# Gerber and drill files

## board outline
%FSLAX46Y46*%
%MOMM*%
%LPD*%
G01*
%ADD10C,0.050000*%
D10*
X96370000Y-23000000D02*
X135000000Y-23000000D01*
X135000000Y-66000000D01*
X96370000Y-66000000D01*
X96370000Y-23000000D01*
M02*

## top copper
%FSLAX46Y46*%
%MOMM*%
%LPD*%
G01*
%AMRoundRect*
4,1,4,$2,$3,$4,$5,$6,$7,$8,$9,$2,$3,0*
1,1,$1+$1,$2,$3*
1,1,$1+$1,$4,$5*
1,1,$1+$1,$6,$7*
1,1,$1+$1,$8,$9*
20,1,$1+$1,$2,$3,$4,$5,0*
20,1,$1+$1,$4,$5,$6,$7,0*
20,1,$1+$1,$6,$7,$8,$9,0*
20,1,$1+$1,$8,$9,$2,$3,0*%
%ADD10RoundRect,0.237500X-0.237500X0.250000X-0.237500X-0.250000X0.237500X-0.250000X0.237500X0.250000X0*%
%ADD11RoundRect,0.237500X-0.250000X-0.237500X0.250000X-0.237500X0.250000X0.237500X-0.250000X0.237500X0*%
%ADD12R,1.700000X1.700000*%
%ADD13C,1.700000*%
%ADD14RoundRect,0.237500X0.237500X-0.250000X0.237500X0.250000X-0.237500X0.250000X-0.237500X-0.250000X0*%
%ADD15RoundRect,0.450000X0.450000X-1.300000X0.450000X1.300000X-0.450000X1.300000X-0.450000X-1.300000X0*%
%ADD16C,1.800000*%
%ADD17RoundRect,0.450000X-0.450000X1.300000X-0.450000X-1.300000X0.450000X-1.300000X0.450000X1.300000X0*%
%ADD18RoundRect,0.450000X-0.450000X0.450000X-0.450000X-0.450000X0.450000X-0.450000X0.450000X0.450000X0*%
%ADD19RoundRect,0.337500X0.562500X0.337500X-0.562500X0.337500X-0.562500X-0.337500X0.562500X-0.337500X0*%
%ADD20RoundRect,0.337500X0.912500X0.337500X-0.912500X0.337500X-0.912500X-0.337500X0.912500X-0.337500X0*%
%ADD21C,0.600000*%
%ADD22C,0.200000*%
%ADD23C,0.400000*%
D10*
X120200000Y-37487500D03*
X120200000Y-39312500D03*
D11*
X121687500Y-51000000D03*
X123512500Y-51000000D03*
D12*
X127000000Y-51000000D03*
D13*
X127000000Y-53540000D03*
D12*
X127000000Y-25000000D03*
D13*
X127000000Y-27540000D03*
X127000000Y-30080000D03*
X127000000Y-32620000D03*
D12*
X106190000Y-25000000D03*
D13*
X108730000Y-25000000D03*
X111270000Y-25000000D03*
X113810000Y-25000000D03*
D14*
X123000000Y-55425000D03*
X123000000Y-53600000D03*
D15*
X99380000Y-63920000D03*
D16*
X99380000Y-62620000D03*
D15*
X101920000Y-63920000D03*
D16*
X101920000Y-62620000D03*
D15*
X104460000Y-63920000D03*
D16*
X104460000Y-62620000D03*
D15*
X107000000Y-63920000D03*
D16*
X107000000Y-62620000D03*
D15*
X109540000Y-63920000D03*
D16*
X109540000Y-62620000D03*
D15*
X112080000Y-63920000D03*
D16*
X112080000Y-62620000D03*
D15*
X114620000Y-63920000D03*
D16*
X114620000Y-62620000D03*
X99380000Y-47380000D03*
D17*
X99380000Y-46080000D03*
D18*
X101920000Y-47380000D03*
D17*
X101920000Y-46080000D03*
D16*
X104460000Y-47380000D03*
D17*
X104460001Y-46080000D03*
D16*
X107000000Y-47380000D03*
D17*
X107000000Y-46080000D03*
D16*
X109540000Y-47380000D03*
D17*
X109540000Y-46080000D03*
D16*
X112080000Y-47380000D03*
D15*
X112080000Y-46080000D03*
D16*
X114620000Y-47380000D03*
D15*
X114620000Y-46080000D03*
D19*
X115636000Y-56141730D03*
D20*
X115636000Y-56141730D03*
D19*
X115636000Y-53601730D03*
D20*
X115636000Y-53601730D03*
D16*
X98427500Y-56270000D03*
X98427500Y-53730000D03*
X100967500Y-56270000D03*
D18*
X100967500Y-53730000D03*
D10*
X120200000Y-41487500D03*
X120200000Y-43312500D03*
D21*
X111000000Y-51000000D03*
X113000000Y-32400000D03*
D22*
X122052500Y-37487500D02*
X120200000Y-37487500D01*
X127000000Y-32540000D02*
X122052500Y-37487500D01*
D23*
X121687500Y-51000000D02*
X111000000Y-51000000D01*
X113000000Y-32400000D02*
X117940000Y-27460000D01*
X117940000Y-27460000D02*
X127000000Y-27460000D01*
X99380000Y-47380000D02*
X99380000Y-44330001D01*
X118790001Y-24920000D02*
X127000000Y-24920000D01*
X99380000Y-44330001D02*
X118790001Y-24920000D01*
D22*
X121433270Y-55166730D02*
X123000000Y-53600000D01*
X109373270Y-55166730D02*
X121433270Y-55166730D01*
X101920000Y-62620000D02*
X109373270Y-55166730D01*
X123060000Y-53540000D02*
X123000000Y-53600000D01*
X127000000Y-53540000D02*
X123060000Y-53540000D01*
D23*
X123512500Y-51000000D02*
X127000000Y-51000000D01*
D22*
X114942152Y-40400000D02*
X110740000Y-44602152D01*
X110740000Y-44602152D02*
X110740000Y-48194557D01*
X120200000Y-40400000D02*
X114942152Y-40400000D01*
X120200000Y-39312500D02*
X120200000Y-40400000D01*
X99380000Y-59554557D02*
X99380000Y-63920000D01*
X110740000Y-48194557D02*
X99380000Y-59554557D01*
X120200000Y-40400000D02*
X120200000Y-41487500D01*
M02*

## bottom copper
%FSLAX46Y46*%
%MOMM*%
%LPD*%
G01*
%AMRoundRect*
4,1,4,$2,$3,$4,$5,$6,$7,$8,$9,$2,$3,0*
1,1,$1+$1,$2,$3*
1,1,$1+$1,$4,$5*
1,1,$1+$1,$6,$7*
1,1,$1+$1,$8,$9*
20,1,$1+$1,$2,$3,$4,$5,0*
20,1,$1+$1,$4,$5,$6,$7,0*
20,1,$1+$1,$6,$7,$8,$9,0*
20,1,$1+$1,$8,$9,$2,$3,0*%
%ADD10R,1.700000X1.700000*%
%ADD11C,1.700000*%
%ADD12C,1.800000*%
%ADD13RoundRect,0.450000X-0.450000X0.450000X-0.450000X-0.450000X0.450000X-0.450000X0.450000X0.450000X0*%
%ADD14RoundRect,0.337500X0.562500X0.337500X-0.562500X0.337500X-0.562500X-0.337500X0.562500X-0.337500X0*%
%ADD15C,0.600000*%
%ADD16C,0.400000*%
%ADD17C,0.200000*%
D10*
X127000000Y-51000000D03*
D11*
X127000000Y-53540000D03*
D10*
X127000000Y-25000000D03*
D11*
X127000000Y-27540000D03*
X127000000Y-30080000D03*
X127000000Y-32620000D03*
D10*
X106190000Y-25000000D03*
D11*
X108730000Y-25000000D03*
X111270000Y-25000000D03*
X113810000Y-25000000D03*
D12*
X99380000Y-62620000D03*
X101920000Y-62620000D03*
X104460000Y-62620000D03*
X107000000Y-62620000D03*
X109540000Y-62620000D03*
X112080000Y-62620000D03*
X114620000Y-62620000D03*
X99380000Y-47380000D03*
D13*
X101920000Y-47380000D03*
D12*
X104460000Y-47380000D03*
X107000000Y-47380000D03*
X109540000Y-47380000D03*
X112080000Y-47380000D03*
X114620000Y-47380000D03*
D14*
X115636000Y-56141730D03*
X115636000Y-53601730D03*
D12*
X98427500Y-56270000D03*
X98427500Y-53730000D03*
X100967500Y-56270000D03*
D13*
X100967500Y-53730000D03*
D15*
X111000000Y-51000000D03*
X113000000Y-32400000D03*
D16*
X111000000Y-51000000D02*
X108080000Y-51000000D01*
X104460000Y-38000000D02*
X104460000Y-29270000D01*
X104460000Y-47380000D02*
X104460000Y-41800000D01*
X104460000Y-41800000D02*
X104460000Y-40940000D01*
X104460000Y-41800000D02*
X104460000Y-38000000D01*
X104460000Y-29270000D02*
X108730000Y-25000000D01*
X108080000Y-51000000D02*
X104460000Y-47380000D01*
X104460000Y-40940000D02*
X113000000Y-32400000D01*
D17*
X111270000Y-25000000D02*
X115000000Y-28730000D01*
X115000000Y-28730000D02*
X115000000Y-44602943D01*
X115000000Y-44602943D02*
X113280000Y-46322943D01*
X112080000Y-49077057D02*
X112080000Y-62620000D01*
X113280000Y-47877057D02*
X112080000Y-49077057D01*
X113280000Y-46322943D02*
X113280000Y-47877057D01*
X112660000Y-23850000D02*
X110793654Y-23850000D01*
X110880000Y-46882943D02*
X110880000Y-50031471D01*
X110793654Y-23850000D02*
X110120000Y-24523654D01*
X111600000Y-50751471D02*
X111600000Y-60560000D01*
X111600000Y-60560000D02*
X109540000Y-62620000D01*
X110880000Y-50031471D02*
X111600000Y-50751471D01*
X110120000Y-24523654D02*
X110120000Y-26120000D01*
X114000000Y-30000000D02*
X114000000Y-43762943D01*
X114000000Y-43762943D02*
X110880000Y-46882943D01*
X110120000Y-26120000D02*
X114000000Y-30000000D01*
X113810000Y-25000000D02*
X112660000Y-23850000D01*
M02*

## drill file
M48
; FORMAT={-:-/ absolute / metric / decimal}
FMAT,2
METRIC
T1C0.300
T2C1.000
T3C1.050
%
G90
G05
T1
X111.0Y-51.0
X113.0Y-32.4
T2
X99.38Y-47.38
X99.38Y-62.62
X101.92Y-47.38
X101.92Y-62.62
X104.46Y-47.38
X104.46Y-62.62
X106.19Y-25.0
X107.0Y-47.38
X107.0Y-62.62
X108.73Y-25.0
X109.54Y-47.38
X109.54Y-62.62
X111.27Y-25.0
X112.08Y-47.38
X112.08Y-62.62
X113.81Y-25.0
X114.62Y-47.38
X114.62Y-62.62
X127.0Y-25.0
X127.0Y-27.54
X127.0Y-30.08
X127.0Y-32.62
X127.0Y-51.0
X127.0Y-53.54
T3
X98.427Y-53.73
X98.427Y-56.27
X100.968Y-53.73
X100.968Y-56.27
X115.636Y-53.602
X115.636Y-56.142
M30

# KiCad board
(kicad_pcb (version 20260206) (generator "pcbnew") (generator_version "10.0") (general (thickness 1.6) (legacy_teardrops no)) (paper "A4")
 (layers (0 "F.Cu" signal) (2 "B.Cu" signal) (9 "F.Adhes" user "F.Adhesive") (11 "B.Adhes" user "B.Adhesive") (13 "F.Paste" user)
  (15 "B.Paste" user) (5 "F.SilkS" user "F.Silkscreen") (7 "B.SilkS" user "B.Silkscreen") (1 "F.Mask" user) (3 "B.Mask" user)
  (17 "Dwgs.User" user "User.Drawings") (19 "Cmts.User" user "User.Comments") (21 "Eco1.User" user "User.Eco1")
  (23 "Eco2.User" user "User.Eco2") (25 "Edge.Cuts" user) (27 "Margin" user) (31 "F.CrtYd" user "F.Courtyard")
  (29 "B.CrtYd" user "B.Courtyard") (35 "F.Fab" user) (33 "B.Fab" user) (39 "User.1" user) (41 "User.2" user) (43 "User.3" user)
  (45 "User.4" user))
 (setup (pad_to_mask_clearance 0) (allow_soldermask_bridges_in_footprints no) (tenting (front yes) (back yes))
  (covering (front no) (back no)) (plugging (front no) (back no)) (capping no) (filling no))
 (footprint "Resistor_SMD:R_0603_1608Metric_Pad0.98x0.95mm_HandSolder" (layer "F.Cu") (at 120.2 38.4 -90)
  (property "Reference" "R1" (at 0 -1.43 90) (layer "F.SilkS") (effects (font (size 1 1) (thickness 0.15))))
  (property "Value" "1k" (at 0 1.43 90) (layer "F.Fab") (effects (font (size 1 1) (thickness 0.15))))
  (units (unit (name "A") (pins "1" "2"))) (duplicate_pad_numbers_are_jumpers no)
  (pad "1" smd roundrect (at -0.9125 0 270) (size 0.975 0.95) (layers "F.Cu" "F.Mask" "F.Paste") (roundrect_rratio 0.25) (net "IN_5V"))
  (pad "2" smd roundrect (at 0.9125 0 270) (size 0.975 0.95) (layers "F.Cu" "F.Mask" "F.Paste") (roundrect_rratio 0.25) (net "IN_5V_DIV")))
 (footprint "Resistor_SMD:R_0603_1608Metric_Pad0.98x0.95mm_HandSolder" (layer "F.Cu") (at 122.6 51)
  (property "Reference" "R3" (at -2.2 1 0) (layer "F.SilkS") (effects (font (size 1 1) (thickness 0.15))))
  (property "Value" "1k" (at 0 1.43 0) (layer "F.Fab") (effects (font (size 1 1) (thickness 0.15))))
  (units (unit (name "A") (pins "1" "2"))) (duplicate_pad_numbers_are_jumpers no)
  (pad "1" smd roundrect (at -0.9125 0) (size 0.975 0.95) (layers "F.Cu" "F.Mask" "F.Paste") (roundrect_rratio 0.25) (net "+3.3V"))
  (pad "2" smd roundrect (at 0.9125 0) (size 0.975 0.95) (layers "F.Cu" "F.Mask" "F.Paste") (roundrect_rratio 0.25) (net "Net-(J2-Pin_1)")))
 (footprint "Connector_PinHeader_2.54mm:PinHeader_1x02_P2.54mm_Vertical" (layer "F.Cu") (at 127 51)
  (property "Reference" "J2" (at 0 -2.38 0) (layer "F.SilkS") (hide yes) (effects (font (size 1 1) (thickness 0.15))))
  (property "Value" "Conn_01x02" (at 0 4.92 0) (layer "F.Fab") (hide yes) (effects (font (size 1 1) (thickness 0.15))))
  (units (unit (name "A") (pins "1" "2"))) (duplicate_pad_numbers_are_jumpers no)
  (pad "1" thru_hole rect (at 0 0) (size 1.7 1.7) (drill 1) (layers "*.Cu" "*.Mask") (remove_unused_layers no) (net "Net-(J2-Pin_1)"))
  (pad "2" thru_hole circle (at 0 2.54) (size 1.7 1.7) (drill 1) (layers "*.Cu" "*.Mask") (remove_unused_layers no) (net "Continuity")))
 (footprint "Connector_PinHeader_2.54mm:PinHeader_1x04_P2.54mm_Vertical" (layer "F.Cu") (at 127 25)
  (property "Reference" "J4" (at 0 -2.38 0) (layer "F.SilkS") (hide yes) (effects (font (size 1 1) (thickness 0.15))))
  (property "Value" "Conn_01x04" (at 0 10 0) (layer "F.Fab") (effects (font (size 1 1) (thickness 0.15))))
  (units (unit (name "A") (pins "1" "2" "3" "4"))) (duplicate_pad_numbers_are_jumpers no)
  (pad "1" thru_hole rect (at 0 0) (size 1.7 1.7) (drill 1) (layers "*.Cu" "*.Mask") (remove_unused_layers no) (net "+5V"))
  (pad "2" thru_hole circle (at 0 2.54) (size 1.7 1.7) (drill 1) (layers "*.Cu" "*.Mask") (remove_unused_layers no) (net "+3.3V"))
  (pad "3" thru_hole circle (at 0 5.08) (size 1.7 1.7) (drill 1) (layers "*.Cu" "*.Mask") (remove_unused_layers no) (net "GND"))
  (pad "4" thru_hole circle (at 0 7.62) (size 1.7 1.7) (drill 1) (layers "*.Cu" "*.Mask") (remove_unused_layers no) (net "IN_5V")))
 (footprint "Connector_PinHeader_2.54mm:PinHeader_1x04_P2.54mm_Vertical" (layer "F.Cu") (at 106.19 25 90)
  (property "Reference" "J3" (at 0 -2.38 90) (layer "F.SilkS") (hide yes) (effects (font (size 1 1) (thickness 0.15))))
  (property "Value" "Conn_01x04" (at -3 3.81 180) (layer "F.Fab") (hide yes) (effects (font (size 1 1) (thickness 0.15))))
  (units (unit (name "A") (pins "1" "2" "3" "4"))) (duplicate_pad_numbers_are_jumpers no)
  (pad "1" thru_hole rect (at 0 0 90) (size 1.7 1.7) (drill 1) (layers "*.Cu" "*.Mask") (remove_unused_layers no) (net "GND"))
  (pad "2" thru_hole circle (at 0 2.54 90) (size 1.7 1.7) (drill 1) (layers "*.Cu" "*.Mask") (remove_unused_layers no) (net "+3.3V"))
  (pad "3" thru_hole circle (at 0 5.08 90) (size 1.7 1.7) (drill 1) (layers "*.Cu" "*.Mask") (remove_unused_layers no) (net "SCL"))
  (pad "4" thru_hole circle (at 0 7.62 90) (size 1.7 1.7) (drill 1) (layers "*.Cu" "*.Mask") (remove_unused_layers no) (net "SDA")))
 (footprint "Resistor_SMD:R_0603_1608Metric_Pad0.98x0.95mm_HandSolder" (layer "F.Cu") (at 123 54.5125 90)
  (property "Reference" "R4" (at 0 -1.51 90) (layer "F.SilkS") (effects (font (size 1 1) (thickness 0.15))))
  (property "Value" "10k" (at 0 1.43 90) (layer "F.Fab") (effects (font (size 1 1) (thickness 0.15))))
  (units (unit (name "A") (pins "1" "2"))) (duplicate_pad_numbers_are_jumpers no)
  (pad "1" smd roundrect (at -0.9125 0 90) (size 0.975 0.95) (layers "F.Cu" "F.Mask" "F.Paste") (roundrect_rratio 0.25) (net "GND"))
  (pad "2" smd roundrect (at 0.9125 0 90) (size 0.975 0.95) (layers "F.Cu" "F.Mask" "F.Paste") (roundrect_rratio 0.25) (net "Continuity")))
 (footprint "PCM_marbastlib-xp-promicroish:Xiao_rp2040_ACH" (layer "F.Cu") (at 107 55 90)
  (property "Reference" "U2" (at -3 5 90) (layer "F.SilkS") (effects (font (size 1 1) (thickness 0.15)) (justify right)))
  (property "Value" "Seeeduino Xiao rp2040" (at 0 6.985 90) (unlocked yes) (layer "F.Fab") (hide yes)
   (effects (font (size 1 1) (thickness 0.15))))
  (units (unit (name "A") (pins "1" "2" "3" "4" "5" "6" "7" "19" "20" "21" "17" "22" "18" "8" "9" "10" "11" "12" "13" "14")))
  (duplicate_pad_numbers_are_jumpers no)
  (pad "1" smd roundrect (at -8.92 -7.62 90) (size 3.5 1.8) (layers "F.Cu" "F.Mask") (roundrect_rratio 0.25) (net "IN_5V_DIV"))
  (pad "1" thru_hole circle (at -7.62 -7.62 90) (size 1.8 1.8) (drill 1) (layers "*.Cu" "*.Mask") (remove_unused_layers no)
   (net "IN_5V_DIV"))
  (pad "2" smd roundrect (at -8.92 -5.08 90) (size 3.5 1.8) (layers "F.Cu" "F.Mask") (roundrect_rratio 0.25) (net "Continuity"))
  (pad "2" thru_hole circle (at -7.62 -5.08 90) (size 1.8 1.8) (drill 1) (layers "*.Cu" "*.Mask") (remove_unused_layers no)
   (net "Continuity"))
  (pad "3" smd roundrect (at -8.92 -2.54 90) (size 3.5 1.8) (layers "F.Cu" "F.Mask") (roundrect_rratio 0.25)
   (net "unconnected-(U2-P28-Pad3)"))
  (pad "3" thru_hole circle (at -7.62 -2.54 90) (size 1.8 1.8) (drill 1) (layers "*.Cu" "*.Mask") (remove_unused_layers no)
   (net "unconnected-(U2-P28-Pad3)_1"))
  (pad "4" smd roundrect (at -8.92 0 90) (size 3.5 1.8) (layers "F.Cu" "F.Mask") (roundrect_rratio 0.25) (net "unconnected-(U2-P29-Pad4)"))
  (pad "4" thru_hole circle (at -7.62 0 90) (size 1.8 1.8) (drill 1) (layers "*.Cu" "*.Mask") (remove_unused_layers no)
   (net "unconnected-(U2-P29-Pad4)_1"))
  (pad "5" smd roundrect (at -8.92 2.54 90) (size 3.5 1.8) (layers "F.Cu" "F.Mask") (roundrect_rratio 0.25) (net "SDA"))
  (pad "5" thru_hole circle (at -7.62 2.54 90) (size 1.8 1.8) (drill 1) (layers "*.Cu" "*.Mask") (remove_unused_layers no) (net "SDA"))
  (pad "6" smd roundrect (at -8.92 5.08 90) (size 3.5 1.8) (layers "F.Cu" "F.Mask") (roundrect_rratio 0.25) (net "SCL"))
  (pad "6" thru_hole circle (at -7.62 5.08 90) (size 1.8 1.8) (drill 1) (layers "*.Cu" "*.Mask") (remove_unused_layers no) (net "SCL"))
  (pad "7" smd roundrect (at -8.92 7.62 90) (size 3.5 1.8) (layers "F.Cu" "F.Mask") (roundrect_rratio 0.25) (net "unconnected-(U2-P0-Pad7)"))
  (pad "7" thru_hole circle (at -7.62 7.62 90) (size 1.8 1.8) (drill 1) (layers "*.Cu" "*.Mask") (remove_unused_layers no)
   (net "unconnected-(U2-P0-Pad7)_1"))
  (pad "8" thru_hole circle (at 7.62 -7.62 270) (size 1.8 1.8) (drill 1) (layers "*.Cu" "*.Mask") (remove_unused_layers no) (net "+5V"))
  (pad "8" smd roundrect (at 8.92 -7.62 270) (size 3.5 1.8) (layers "F.Cu" "F.Mask") (roundrect_rratio 0.25) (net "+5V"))
  (pad "9" thru_hole roundrect (at 7.62 -5.08 270) (size 1.8 1.8) (drill 1) (layers "*.Cu" "*.Mask") (remove_unused_layers no)
   (roundrect_rratio 0.25) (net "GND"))
  (pad "9" smd roundrect (at 8.92 -5.08 270) (size 3.5 1.8) (layers "F.Cu" "F.Mask") (roundrect_rratio 0.25) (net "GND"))
  (pad "10" thru_hole circle (at 7.62 -2.54 270) (size 1.8 1.8) (drill 1) (layers "*.Cu" "*.Mask") (remove_unused_layers no) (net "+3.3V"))
  (pad "10" smd roundrect (at 8.92 -2.539999 270) (size 3.5 1.8) (layers "F.Cu" "F.Mask") (roundrect_rratio 0.25) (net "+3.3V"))
  (pad "11" thru_hole circle (at 7.62 0 270) (size 1.8 1.8) (drill 1) (layers "*.Cu" "*.Mask") (remove_unused_layers no)
   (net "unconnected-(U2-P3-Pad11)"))
  (pad "11" smd roundrect (at 8.92 0 270) (size 3.5 1.8) (layers "F.Cu" "F.Mask") (roundrect_rratio 0.25)
   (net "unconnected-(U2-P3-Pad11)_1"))
  (pad "12" thru_hole circle (at 7.62 2.54 270) (size 1.8 1.8) (drill 1) (layers "*.Cu" "*.Mask") (remove_unused_layers no)
   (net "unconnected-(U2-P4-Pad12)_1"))
  (pad "12" smd roundrect (at 8.92 2.54 270) (size 3.5 1.8) (layers "F.Cu" "F.Mask") (roundrect_rratio 0.25)
   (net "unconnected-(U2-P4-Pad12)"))
  (pad "13" thru_hole circle (at 7.62 5.08 90) (size 1.8 1.8) (drill 1) (layers "*.Cu" "*.Mask") (remove_unused_layers no)
   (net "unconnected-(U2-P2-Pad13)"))
  (pad "13" smd roundrect (at 8.92 5.08 90) (size 3.5 1.8) (layers "F.Cu" "F.Mask") (roundrect_rratio 0.25)
   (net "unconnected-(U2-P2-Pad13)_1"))
  (pad "14" thru_hole circle (at 7.62 7.62 90) (size 1.8 1.8) (drill 1) (layers "*.Cu" "*.Mask") (remove_unused_layers no)
   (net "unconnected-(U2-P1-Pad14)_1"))
  (pad "14" smd roundrect (at 8.92 7.62 90) (size 3.5 1.8) (layers "F.Cu" "F.Mask") (roundrect_rratio 0.25)
   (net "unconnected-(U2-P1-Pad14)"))
  (pad "17" thru_hole roundrect (at -1.14173 8.636 180) (size 1.8 1.35) (drill 1.05) (layers "*.Cu" "*.Mask") (remove_unused_layers no)
   (roundrect_rratio 0.25) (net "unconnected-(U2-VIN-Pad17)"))
  (pad "17" smd roundrect (at -1.14173 8.636 180) (size 2.5 1.35) (layers "F.Cu" "F.Mask") (roundrect_rratio 0.25)
   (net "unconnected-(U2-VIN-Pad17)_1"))
  (pad "18" thru_hole roundrect (at 1.39827 8.636 180) (size 1.8 1.35) (drill 1.05) (layers "*.Cu" "*.Mask") (remove_unused_layers no)
   (roundrect_rratio 0.25) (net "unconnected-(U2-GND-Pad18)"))
  (pad "18" smd roundrect (at 1.39827 8.636 180) (size 2.5 1.35) (layers "F.Cu" "F.Mask") (roundrect_rratio 0.25)
   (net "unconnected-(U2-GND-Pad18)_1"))
  (pad "19" thru_hole circle (at -1.27 -8.5725 270) (size 1.8 1.8) (drill 1.05) (layers "*.Cu" "*.Mask") (remove_unused_layers no)
   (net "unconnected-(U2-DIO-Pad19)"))
  (pad "20" thru_hole circle (at 1.27 -8.5725 270) (size 1.8 1.8) (drill 1.05) (layers "*.Cu" "*.Mask") (remove_unused_layers no)
   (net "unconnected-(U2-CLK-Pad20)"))
  (pad "21" thru_hole circle (at -1.27 -6.0325 270) (size 1.8 1.8) (drill 1.05) (layers "*.Cu" "*.Mask") (remove_unused_layers no)
   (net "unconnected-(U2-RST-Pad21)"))
  (pad "22" thru_hole roundrect (at 1.27 -6.0325 270) (size 1.8 1.8) (drill 1.05) (layers "*.Cu" "*.Mask") (remove_unused_layers no)
   (roundrect_rratio 0.25) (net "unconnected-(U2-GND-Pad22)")))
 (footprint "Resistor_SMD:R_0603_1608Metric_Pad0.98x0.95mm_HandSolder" (layer "F.Cu") (at 120.2 42.4 -90)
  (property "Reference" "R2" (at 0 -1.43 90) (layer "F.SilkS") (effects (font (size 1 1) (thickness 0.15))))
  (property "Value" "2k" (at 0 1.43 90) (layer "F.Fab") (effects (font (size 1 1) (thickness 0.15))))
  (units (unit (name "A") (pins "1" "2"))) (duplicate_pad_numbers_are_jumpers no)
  (pad "1" smd roundrect (at -0.9125 0 270) (size 0.975 0.95) (layers "F.Cu" "F.Mask" "F.Paste") (roundrect_rratio 0.25) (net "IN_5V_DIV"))
  (pad "2" smd roundrect (at 0.9125 0 270) (size 0.975 0.95) (layers "F.Cu" "F.Mask" "F.Paste") (roundrect_rratio 0.25) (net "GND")))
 (gr_rect (start 96.37 23) (end 135 66) (stroke (width 0.05) (type default)) (fill no) (layer "Edge.Cuts"))
 (segment (start 122.0525 37.4875) (end 120.2 37.4875) (width 0.2) (layer "F.Cu") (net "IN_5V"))
 (segment (start 127 32.54) (end 122.0525 37.4875) (width 0.2) (layer "F.Cu") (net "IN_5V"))
 (segment (start 121.6875 51) (end 111 51) (width 0.4) (layer "F.Cu") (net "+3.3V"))
 (segment (start 113 32.4) (end 117.94 27.46) (width 0.4) (layer "F.Cu") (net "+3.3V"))
 (segment (start 117.94 27.46) (end 127 27.46) (width 0.4) (layer "F.Cu") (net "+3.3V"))
 (via (at 111 51) (size 0.6) (drill 0.3) (layers "F.Cu" "B.Cu") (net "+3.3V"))
 (via (at 113 32.4) (size 0.6) (drill 0.3) (layers "F.Cu" "B.Cu") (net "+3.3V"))
 (segment (start 111 51) (end 108.08 51) (width 0.4) (layer "B.Cu") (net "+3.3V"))
 (segment (start 104.46 38) (end 104.46 29.27) (width 0.4) (layer "B.Cu") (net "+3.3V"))
 (segment (start 104.46 47.38) (end 104.46 41.8) (width 0.4) (layer "B.Cu") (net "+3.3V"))
 (segment (start 104.46 41.8) (end 104.46 40.94) (width 0.4) (layer "B.Cu") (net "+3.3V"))
 (segment (start 104.46 41.8) (end 104.46 38) (width 0.4) (layer "B.Cu") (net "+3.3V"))
 (segment (start 104.46 29.27) (end 108.73 25) (width 0.4) (layer "B.Cu") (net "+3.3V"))
 (segment (start 108.08 51) (end 104.46 47.38) (width 0.4) (layer "B.Cu") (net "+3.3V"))
 (segment (start 104.46 40.94) (end 113 32.4) (width 0.4) (layer "B.Cu") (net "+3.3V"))
 (segment (start 99.38 47.38) (end 99.38 44.330001) (width 0.4) (layer "F.Cu") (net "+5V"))
 (segment (start 118.790001 24.92) (end 127 24.92) (width 0.4) (layer "F.Cu") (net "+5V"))
 (segment (start 99.38 44.330001) (end 118.790001 24.92) (width 0.4) (layer "F.Cu") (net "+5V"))
 (segment (start 121.43327 55.16673) (end 123 53.6) (width 0.2) (layer "F.Cu") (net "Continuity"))
 (segment (start 109.37327 55.16673) (end 121.43327 55.16673) (width 0.2) (layer "F.Cu") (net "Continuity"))
 (segment (start 101.92 62.62) (end 109.37327 55.16673) (width 0.2) (layer "F.Cu") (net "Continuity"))
 (segment (start 123.06 53.54) (end 123 53.6) (width 0.2) (layer "F.Cu") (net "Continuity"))
 (segment (start 127 53.54) (end 123.06 53.54) (width 0.2) (layer "F.Cu") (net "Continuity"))
 (segment (start 123.5125 51) (end 127 51) (width 0.4) (layer "F.Cu") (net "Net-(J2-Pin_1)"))
 (segment (start 111.27 25) (end 115 28.73) (width 0.2) (layer "B.Cu") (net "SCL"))
 (segment (start 115 28.73) (end 115 44.602943) (width 0.2) (layer "B.Cu") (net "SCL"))
 (segment (start 115 44.602943) (end 113.28 46.322943) (width 0.2) (layer "B.Cu") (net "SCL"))
 (segment (start 112.08 49.077057) (end 112.08 62.62) (width 0.2) (layer "B.Cu") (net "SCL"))
 (segment (start 113.28 47.877057) (end 112.08 49.077057) (width 0.2) (layer "B.Cu") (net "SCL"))
 (segment (start 113.28 46.322943) (end 113.28 47.877057) (width 0.2) (layer "B.Cu") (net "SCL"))
 (segment (start 112.66 23.85) (end 110.793654 23.85) (width 0.2) (layer "B.Cu") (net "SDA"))
 (segment (start 110.88 46.882943) (end 110.88 50.031471) (width 0.2) (layer "B.Cu") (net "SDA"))
 (segment (start 110.793654 23.85) (end 110.12 24.523654) (width 0.2) (layer "B.Cu") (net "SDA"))
 (segment (start 111.6 50.751471) (end 111.6 60.56) (width 0.2) (layer "B.Cu") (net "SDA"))
 (segment (start 111.6 60.56) (end 109.54 62.62) (width 0.2) (layer "B.Cu") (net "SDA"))
 (segment (start 110.88 50.031471) (end 111.6 50.751471) (width 0.2) (layer "B.Cu") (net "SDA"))
 (segment (start 110.12 24.523654) (end 110.12 26.12) (width 0.2) (layer "B.Cu") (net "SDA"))
 (segment (start 114 30) (end 114 43.762943) (width 0.2) (layer "B.Cu") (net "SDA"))
 (segment (start 114 43.762943) (end 110.88 46.882943) (width 0.2) (layer "B.Cu") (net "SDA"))
 (segment (start 110.12 26.12) (end 114 30) (width 0.2) (layer "B.Cu") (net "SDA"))
 (segment (start 113.81 25) (end 112.66 23.85) (width 0.2) (layer "B.Cu") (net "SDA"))
 (segment (start 114.942152 40.4) (end 110.74 44.602152) (width 0.2) (layer "F.Cu") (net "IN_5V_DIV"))
 (segment (start 110.74 44.602152) (end 110.74 48.194557) (width 0.2) (layer "F.Cu") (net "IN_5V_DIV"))
 (segment (start 120.2 40.4) (end 114.942152 40.4) (width 0.2) (layer "F.Cu") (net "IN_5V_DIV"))
 (segment (start 120.2 39.3125) (end 120.2 40.4) (width 0.2) (layer "F.Cu") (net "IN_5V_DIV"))
 (segment (start 99.38 59.554557) (end 99.38 63.92) (width 0.2) (layer "F.Cu") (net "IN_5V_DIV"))
 (segment (start 110.74 48.194557) (end 99.38 59.554557) (width 0.2) (layer "F.Cu") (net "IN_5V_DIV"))
 (segment (start 120.2 40.4) (end 120.2 41.4875) (width 0.2) (layer "F.Cu") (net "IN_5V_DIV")))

